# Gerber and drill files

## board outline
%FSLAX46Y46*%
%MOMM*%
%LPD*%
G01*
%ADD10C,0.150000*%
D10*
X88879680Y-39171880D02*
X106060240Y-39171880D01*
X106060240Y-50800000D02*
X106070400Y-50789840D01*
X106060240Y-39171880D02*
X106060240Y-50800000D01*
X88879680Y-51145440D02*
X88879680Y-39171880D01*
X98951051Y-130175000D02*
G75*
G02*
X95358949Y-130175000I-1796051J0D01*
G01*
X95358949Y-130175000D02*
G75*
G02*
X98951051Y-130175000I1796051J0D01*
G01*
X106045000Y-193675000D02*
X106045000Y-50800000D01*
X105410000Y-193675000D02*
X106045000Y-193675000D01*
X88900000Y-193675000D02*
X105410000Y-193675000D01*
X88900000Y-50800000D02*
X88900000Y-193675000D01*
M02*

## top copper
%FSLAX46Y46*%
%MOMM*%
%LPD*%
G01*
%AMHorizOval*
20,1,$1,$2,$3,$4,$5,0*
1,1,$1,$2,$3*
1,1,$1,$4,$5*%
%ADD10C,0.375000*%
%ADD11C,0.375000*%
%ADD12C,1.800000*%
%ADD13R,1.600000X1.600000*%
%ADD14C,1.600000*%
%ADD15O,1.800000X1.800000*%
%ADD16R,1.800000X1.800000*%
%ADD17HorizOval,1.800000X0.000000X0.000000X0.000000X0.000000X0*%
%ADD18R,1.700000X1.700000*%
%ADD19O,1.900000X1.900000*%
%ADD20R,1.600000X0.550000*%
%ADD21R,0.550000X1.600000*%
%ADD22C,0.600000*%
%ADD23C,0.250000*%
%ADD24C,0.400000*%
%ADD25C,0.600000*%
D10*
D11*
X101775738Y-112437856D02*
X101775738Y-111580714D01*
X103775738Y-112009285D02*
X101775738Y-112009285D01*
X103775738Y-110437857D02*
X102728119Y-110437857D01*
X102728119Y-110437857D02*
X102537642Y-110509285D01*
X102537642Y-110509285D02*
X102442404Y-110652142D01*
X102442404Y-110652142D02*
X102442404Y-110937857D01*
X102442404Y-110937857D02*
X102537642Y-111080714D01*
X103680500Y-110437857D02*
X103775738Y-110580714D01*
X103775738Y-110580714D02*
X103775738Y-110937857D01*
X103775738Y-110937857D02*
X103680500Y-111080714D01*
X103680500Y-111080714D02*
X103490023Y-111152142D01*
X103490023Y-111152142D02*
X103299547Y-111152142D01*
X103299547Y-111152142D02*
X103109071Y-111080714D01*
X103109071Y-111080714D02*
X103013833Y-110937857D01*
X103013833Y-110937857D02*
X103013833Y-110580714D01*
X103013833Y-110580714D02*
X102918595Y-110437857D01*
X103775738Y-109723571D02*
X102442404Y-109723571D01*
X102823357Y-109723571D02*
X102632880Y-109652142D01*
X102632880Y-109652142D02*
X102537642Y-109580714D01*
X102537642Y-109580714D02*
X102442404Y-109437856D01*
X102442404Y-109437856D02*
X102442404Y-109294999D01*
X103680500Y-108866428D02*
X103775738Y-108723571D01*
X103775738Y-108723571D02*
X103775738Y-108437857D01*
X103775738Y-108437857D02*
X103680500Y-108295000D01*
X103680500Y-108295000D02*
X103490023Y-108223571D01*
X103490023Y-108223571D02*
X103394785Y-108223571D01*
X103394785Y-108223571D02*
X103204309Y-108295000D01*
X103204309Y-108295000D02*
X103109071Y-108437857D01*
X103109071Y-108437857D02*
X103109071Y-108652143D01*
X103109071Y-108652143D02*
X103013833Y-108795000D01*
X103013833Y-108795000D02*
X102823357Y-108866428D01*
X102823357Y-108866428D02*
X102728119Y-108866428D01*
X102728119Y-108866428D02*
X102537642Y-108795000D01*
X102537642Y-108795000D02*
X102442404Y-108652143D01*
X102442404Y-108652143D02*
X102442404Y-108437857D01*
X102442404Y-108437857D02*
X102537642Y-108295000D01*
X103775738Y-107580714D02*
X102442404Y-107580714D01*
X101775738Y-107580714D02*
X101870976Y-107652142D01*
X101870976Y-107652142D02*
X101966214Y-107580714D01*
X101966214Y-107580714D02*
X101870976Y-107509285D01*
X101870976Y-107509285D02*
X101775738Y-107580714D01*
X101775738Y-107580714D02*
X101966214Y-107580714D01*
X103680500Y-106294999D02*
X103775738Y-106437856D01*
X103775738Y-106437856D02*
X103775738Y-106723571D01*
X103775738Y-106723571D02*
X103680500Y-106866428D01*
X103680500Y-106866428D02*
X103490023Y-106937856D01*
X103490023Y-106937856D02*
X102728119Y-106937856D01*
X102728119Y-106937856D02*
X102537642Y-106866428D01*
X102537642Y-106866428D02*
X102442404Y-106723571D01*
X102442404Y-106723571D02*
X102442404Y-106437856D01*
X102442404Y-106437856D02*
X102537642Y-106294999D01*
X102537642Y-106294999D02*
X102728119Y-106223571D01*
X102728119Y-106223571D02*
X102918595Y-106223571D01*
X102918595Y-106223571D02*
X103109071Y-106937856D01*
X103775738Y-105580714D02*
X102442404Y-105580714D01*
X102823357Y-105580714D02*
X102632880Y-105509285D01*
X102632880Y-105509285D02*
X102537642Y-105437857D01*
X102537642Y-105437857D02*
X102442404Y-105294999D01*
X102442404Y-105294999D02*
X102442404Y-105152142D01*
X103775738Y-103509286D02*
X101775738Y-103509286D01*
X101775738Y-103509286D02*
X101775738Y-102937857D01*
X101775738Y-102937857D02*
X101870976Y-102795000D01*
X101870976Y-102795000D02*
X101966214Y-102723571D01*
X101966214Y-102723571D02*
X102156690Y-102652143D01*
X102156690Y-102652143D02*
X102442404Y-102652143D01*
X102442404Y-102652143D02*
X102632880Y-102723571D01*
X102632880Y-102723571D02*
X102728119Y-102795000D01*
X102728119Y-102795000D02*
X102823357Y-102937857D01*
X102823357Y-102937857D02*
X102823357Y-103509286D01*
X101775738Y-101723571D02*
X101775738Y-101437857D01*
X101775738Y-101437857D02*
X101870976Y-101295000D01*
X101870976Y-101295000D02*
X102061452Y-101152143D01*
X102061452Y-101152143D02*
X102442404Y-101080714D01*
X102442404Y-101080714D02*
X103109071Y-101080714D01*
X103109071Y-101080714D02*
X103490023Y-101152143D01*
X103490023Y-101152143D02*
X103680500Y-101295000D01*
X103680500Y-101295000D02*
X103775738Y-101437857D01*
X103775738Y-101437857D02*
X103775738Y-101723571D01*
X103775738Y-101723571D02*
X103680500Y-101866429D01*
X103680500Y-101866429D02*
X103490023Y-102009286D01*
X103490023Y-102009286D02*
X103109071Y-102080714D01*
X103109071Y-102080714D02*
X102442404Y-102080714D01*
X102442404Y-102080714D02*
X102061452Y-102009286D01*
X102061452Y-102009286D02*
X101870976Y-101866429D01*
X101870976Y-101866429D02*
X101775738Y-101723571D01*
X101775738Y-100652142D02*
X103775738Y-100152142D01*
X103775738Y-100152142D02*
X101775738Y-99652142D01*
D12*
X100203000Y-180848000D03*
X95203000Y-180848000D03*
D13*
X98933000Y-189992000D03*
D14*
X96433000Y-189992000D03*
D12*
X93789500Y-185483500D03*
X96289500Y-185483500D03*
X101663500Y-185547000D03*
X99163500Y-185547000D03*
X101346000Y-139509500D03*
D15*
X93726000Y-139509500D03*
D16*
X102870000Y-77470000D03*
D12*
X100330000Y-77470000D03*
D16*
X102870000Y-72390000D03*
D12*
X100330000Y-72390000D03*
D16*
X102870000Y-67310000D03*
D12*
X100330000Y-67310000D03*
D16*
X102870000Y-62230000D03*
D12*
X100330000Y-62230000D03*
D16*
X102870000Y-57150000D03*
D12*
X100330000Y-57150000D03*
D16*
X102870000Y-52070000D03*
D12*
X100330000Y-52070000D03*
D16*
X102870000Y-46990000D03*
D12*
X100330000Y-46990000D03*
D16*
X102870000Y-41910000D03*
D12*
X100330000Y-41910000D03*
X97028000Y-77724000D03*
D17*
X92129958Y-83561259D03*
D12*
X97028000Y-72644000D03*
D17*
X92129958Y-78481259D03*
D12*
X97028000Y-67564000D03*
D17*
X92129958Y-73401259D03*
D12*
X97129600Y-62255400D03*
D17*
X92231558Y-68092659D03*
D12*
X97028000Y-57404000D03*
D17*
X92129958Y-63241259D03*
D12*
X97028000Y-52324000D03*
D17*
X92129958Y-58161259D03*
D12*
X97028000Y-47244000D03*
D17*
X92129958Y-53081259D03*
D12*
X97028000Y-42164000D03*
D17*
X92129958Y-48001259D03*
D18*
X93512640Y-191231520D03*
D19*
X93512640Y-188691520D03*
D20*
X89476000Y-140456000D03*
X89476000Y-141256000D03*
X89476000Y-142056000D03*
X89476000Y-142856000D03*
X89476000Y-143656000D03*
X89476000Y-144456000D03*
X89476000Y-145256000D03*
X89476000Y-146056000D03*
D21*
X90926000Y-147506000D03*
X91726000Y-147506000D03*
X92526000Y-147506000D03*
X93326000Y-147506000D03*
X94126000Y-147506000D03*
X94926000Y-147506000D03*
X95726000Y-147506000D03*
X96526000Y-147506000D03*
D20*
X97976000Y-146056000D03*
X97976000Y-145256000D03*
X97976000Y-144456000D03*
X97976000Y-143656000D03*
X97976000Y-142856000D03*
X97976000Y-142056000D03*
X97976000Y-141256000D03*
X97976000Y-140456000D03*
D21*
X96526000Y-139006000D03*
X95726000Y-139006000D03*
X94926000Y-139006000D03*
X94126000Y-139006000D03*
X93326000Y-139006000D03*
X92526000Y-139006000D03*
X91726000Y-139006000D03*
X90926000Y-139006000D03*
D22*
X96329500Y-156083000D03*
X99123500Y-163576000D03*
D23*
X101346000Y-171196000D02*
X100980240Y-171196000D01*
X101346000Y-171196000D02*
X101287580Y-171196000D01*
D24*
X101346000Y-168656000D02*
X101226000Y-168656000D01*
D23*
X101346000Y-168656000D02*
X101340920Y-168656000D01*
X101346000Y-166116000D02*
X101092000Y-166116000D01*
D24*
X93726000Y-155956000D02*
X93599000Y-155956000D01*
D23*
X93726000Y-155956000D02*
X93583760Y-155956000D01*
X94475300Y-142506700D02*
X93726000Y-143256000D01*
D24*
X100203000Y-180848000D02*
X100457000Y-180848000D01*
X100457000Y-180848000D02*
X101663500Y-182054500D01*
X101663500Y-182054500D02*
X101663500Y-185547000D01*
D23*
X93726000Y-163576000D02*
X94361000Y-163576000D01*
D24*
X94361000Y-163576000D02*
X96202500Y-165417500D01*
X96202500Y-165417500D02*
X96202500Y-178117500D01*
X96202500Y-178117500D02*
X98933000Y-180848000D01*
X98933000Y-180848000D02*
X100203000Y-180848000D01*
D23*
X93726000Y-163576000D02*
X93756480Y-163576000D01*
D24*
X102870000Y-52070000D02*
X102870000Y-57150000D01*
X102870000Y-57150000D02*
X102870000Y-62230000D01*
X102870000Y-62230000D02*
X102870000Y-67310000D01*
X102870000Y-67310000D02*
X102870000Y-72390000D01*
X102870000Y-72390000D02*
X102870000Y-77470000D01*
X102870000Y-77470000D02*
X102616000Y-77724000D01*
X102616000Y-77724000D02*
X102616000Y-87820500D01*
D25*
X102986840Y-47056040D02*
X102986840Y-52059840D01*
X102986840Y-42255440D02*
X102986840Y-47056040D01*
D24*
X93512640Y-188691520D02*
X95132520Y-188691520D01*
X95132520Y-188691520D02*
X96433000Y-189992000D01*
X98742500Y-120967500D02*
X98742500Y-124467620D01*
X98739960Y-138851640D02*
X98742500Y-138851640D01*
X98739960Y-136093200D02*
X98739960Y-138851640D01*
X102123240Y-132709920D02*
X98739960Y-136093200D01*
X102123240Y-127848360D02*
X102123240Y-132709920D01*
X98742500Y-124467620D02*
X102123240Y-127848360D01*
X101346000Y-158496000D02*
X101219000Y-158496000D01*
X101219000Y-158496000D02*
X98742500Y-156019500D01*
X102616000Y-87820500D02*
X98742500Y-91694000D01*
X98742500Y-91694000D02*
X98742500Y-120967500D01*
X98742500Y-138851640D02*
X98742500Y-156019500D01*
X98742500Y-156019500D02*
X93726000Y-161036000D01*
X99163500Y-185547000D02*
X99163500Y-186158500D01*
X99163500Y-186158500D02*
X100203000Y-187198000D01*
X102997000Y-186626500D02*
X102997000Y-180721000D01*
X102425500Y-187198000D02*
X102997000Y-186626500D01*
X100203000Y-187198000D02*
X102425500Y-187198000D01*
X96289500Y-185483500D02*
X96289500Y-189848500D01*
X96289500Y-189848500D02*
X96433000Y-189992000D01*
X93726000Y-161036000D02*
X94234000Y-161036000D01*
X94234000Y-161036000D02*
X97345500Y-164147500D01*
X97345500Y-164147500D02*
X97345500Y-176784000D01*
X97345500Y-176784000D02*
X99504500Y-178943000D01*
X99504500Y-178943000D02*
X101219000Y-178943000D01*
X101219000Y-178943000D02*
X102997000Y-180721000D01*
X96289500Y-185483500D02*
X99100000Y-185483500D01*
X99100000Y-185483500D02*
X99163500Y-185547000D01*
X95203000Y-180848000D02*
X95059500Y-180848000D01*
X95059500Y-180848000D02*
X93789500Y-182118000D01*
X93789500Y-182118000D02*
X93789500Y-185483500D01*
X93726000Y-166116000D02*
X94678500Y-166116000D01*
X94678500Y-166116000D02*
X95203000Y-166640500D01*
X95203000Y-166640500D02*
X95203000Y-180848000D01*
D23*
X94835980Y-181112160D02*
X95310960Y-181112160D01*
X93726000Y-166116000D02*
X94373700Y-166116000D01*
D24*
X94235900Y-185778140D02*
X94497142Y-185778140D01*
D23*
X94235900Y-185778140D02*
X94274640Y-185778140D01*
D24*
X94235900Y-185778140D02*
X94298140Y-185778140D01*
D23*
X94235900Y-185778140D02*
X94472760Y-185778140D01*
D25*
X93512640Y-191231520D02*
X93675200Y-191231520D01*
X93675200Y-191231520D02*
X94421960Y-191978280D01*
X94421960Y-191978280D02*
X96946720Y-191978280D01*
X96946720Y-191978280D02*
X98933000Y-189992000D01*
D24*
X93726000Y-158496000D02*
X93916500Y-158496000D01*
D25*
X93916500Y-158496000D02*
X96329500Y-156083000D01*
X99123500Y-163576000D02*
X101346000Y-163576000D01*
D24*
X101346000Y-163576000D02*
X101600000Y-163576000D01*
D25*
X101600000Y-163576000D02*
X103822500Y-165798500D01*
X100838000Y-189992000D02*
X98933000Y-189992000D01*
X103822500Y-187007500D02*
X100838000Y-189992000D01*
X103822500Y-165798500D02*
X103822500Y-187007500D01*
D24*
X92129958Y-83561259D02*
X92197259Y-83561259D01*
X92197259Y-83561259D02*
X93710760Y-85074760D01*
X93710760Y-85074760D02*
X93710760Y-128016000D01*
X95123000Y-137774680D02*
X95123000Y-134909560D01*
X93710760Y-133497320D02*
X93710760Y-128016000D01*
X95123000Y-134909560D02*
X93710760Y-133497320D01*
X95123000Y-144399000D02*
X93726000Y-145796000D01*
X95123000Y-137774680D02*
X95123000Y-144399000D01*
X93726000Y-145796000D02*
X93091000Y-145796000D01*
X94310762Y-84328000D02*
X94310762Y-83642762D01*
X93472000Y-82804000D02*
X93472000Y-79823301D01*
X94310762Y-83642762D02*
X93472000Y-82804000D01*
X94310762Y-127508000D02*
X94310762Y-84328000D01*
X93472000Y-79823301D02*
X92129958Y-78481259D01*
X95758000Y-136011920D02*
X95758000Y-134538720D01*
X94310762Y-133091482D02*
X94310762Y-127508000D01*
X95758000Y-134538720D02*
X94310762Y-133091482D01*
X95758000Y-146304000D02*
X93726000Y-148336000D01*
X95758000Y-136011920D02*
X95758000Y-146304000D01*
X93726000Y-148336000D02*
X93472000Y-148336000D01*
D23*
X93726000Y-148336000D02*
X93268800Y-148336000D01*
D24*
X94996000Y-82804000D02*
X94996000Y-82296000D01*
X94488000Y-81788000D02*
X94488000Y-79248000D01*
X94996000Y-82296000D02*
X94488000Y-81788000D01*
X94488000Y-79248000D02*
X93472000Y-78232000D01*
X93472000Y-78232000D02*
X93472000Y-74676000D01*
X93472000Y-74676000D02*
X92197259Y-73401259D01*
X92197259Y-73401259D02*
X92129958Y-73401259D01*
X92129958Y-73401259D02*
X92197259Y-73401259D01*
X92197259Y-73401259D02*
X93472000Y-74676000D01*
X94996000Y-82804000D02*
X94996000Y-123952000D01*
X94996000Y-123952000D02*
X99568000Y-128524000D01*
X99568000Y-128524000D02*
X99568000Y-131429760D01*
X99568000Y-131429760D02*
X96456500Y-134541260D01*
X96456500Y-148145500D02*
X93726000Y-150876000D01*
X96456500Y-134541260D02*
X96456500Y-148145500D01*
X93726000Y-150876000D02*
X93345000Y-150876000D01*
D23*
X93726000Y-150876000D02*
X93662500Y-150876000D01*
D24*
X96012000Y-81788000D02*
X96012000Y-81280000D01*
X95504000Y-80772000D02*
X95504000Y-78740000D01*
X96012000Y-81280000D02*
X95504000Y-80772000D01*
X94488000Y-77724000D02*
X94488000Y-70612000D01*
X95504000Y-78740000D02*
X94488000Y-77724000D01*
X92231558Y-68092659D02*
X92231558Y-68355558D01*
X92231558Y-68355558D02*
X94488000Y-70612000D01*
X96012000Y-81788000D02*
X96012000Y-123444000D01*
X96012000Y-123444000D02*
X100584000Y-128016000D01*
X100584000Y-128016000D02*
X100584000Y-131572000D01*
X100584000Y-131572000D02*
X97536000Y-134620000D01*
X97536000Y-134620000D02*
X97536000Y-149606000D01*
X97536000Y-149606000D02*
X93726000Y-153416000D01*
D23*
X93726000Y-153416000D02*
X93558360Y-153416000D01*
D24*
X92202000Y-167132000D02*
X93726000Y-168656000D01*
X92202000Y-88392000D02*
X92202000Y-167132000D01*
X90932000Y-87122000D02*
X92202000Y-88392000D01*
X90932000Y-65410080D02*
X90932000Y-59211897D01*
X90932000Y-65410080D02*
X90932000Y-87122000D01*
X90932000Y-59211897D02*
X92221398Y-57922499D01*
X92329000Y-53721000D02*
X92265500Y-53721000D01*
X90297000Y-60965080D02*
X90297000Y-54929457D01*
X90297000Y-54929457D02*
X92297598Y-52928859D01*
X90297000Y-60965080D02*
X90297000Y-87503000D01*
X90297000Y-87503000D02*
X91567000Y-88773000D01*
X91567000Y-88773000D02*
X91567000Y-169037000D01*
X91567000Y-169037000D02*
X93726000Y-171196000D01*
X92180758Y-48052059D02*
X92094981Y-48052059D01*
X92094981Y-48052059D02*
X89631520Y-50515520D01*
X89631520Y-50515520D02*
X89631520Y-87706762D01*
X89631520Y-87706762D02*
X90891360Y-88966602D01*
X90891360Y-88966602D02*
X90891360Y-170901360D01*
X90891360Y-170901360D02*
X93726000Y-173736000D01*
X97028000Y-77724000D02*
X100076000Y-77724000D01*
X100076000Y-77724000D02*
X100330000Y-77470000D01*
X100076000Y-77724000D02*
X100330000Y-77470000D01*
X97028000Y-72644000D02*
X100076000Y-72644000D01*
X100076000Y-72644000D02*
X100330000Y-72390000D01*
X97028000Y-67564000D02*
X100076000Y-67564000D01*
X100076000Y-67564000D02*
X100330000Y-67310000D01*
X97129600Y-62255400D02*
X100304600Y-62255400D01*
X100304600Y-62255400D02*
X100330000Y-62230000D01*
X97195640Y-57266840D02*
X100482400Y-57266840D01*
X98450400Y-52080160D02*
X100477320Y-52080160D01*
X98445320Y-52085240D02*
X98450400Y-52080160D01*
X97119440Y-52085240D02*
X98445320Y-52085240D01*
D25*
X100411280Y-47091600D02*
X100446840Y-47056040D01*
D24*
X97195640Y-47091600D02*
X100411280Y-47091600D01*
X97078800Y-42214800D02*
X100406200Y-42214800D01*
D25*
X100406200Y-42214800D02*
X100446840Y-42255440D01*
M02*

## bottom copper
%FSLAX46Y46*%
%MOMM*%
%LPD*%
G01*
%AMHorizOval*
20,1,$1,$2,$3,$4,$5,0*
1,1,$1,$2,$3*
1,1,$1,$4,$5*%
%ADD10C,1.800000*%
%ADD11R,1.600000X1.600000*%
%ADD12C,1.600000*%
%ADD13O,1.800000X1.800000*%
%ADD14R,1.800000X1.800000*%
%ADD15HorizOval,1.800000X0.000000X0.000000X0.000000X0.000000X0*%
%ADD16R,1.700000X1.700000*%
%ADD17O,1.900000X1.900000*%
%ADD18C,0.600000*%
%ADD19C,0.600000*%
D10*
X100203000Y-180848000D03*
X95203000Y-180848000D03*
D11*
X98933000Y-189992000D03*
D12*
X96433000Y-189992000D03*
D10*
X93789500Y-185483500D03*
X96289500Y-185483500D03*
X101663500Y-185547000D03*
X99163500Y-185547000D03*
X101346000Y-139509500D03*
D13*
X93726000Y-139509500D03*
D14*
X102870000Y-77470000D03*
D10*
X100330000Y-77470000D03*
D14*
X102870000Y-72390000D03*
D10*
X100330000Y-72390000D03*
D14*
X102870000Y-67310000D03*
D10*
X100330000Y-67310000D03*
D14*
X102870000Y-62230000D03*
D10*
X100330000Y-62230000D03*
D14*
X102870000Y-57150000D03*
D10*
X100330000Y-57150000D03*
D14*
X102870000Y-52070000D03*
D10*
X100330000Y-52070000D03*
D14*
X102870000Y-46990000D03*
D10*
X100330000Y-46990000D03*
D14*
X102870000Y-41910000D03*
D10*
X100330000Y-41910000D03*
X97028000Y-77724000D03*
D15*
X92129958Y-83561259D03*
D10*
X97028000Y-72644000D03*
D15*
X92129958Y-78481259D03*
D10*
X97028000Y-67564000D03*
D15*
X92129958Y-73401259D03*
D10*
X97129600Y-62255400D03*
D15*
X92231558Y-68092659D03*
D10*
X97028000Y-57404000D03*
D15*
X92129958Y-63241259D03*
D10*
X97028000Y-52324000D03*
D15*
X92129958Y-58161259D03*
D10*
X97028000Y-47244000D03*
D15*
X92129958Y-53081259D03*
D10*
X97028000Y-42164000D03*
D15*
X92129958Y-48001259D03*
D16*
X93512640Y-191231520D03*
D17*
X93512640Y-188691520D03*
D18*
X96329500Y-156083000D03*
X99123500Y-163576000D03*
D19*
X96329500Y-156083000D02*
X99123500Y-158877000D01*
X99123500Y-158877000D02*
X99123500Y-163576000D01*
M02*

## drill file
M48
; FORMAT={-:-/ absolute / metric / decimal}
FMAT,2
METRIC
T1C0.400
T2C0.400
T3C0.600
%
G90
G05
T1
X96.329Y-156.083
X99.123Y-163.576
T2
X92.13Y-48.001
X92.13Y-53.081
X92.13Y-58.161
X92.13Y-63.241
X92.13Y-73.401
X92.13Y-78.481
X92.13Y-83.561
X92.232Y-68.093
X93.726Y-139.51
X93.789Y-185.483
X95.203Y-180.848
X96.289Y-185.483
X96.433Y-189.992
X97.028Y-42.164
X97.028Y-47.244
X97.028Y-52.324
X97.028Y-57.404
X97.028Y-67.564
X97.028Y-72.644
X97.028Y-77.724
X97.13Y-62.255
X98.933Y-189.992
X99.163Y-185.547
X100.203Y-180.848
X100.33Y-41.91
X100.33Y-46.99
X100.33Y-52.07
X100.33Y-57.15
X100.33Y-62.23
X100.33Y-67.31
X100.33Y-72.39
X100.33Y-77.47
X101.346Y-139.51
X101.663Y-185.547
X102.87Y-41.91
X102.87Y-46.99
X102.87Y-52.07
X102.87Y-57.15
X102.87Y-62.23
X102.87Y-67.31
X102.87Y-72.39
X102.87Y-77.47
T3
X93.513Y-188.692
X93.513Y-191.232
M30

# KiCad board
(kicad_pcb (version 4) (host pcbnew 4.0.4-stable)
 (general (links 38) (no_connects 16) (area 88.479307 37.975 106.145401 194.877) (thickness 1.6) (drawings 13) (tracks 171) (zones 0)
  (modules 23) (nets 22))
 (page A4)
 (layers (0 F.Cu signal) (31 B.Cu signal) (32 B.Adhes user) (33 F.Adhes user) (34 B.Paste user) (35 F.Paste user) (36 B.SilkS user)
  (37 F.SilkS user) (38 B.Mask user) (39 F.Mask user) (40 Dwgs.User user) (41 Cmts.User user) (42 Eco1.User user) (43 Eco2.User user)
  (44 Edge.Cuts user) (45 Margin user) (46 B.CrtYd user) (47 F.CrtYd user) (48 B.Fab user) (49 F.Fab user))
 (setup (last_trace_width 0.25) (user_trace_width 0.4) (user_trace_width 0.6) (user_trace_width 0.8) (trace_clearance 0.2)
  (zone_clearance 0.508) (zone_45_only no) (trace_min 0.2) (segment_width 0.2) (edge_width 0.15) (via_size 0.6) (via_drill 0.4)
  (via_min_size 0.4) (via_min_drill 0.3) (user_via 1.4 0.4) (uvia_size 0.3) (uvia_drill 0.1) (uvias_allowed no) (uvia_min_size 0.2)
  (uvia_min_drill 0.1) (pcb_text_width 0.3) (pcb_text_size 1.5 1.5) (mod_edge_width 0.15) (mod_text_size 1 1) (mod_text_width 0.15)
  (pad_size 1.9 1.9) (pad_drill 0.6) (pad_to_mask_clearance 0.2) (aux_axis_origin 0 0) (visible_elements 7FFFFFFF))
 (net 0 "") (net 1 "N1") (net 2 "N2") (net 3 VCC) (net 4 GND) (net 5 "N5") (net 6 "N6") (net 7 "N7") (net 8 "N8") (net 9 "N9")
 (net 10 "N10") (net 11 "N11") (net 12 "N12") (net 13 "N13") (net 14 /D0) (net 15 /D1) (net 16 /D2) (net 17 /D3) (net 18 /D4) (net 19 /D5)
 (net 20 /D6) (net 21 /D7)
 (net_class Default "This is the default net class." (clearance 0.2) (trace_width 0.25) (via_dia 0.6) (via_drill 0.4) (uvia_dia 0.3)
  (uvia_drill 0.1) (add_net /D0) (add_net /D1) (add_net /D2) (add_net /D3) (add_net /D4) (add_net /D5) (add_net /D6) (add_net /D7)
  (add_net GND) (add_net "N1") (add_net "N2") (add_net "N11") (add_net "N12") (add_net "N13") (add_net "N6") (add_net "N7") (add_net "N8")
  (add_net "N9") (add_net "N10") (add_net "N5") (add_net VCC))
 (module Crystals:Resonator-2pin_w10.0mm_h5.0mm (layer F.Cu) (at 100.203 180.848 180)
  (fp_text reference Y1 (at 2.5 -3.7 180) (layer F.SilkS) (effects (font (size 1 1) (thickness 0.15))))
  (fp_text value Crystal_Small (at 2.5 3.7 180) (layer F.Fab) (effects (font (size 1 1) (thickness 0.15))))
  (pad 1 thru_hole circle (at 0 0 180) (size 1.8 1.8) (drill 0.4) (layers *.Cu *.Mask) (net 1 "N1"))
  (pad 2 thru_hole circle (at 5 0 180) (size 1.8 1.8) (drill 0.4) (layers *.Cu *.Mask) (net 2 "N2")))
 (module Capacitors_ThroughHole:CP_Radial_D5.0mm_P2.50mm (layer F.Cu) (at 98.933 189.992 180)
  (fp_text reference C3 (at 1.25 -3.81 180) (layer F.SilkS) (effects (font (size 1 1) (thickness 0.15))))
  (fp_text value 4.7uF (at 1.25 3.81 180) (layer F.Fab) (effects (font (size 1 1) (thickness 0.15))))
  (pad 1 thru_hole rect (at 0 0 180) (size 1.6 1.6) (drill 0.4) (layers *.Cu *.Mask) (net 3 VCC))
  (pad 2 thru_hole circle (at 2.5 0 180) (size 1.6 1.6) (drill 0.4) (layers *.Cu *.Mask) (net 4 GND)))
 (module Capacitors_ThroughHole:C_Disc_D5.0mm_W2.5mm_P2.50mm (layer F.Cu) (at 93.7895 185.4835)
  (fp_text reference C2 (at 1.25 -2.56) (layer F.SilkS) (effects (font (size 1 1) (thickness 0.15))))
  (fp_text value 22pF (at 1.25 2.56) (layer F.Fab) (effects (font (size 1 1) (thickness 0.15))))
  (pad 1 thru_hole circle (at 0 0) (size 1.8 1.8) (drill 0.4) (layers *.Cu *.Mask) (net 2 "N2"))
  (pad 2 thru_hole circle (at 2.5 0) (size 1.8 1.8) (drill 0.4) (layers *.Cu *.Mask) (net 4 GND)))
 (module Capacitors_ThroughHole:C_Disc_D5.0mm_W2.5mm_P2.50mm (layer F.Cu) (at 101.6635 185.547 180)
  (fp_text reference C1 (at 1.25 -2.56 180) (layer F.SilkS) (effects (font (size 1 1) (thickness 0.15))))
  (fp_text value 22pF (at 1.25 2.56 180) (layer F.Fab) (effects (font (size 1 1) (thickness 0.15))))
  (pad 1 thru_hole circle (at 0 0 180) (size 1.8 1.8) (drill 0.4) (layers *.Cu *.Mask) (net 1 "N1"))
  (pad 2 thru_hole circle (at 2.5 0 180) (size 1.8 1.8) (drill 0.4) (layers *.Cu *.Mask) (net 4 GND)))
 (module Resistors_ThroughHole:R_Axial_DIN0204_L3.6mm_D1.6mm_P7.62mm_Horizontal (layer F.Cu) (at 101.346 139.5095 180)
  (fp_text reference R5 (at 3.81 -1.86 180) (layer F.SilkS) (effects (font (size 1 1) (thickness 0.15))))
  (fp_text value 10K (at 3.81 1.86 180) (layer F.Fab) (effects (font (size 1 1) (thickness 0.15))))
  (pad 1 thru_hole circle (at 0 0 180) (size 1.8 1.8) (drill 0.4) (layers *.Cu *.Mask) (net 3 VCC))
  (pad 2 thru_hole oval (at 7.62 0 180) (size 1.8 1.8) (drill 0.4) (layers *.Cu *.Mask) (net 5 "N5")))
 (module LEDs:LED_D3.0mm (layer F.Cu) (at 102.87 77.47 180)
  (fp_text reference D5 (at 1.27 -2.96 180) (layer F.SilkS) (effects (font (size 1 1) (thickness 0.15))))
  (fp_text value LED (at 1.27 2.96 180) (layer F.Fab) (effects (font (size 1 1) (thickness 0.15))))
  (pad 1 thru_hole rect (at 0 0 180) (size 1.8 1.8) (drill 0.4) (layers *.Cu *.Mask) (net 4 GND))
  (pad 2 thru_hole circle (at 2.54 0 180) (size 1.8 1.8) (drill 0.4) (layers *.Cu *.Mask) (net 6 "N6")))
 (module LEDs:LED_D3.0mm (layer F.Cu) (at 102.87 72.39 180)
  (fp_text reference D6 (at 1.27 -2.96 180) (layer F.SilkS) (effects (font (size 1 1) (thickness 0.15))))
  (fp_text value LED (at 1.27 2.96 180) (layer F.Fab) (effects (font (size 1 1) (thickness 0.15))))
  (pad 1 thru_hole rect (at 0 0 180) (size 1.8 1.8) (drill 0.4) (layers *.Cu *.Mask) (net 4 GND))
  (pad 2 thru_hole circle (at 2.54 0 180) (size 1.8 1.8) (drill 0.4) (layers *.Cu *.Mask) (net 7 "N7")))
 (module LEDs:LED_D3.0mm (layer F.Cu) (at 102.87 67.31 180)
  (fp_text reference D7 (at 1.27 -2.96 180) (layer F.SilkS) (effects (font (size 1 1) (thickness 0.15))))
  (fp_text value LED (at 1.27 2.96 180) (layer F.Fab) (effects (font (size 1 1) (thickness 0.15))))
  (pad 1 thru_hole rect (at 0 0 180) (size 1.8 1.8) (drill 0.4) (layers *.Cu *.Mask) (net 4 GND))
  (pad 2 thru_hole circle (at 2.54 0 180) (size 1.8 1.8) (drill 0.4) (layers *.Cu *.Mask) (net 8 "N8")))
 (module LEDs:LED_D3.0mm (layer F.Cu) (at 102.87 62.23 180)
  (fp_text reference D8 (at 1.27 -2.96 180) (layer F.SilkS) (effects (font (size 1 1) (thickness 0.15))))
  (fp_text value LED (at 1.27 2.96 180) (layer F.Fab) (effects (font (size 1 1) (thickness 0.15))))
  (pad 1 thru_hole rect (at 0 0 180) (size 1.8 1.8) (drill 0.4) (layers *.Cu *.Mask) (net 4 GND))
  (pad 2 thru_hole circle (at 2.54 0 180) (size 1.8 1.8) (drill 0.4) (layers *.Cu *.Mask) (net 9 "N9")))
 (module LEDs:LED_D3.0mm (layer F.Cu) (at 102.87 57.15 180)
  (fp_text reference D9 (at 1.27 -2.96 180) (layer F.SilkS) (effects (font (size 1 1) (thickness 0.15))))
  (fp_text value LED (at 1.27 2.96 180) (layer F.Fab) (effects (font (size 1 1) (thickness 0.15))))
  (pad 1 thru_hole rect (at 0 0 180) (size 1.8 1.8) (drill 0.4) (layers *.Cu *.Mask) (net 4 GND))
  (pad 2 thru_hole circle (at 2.54 0 180) (size 1.8 1.8) (drill 0.4) (layers *.Cu *.Mask) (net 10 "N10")))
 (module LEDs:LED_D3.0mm (layer F.Cu) (at 102.87 52.07 180)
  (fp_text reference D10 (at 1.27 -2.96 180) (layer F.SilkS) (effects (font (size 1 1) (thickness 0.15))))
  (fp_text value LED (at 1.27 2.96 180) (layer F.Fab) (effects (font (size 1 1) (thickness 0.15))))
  (pad 1 thru_hole rect (at 0 0 180) (size 1.8 1.8) (drill 0.4) (layers *.Cu *.Mask) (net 4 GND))
  (pad 2 thru_hole circle (at 2.54 0 180) (size 1.8 1.8) (drill 0.4) (layers *.Cu *.Mask) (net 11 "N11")))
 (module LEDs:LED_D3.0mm (layer F.Cu) (at 102.87 46.99 180)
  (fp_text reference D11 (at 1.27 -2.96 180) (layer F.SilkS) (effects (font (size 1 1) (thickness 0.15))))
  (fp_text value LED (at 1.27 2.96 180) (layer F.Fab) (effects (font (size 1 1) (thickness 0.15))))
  (pad 1 thru_hole rect (at 0 0 180) (size 1.8 1.8) (drill 0.4) (layers *.Cu *.Mask) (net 4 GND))
  (pad 2 thru_hole circle (at 2.54 0 180) (size 1.8 1.8) (drill 0.4) (layers *.Cu *.Mask) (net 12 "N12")))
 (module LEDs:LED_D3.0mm (layer F.Cu) (at 102.87 41.91 180)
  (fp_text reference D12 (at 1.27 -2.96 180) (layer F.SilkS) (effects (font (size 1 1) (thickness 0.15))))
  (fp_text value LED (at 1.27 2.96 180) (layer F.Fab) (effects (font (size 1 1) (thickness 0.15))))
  (pad 1 thru_hole rect (at 0 0 180) (size 1.8 1.8) (drill 0.4) (layers *.Cu *.Mask) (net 4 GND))
  (pad 2 thru_hole circle (at 2.54 0 180) (size 1.8 1.8) (drill 0.4) (layers *.Cu *.Mask) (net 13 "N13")))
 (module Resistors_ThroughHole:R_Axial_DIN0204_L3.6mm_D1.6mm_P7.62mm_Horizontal (layer F.Cu) (at 97.028 77.724 230)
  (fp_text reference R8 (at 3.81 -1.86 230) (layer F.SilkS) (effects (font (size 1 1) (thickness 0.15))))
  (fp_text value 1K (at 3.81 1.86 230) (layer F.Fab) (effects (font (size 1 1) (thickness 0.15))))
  (pad 1 thru_hole circle (at 0 0 230) (size 1.8 1.8) (drill 0.4) (layers *.Cu *.Mask) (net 6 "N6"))
  (pad 2 thru_hole oval (at 7.62 0 230) (size 1.8 1.8) (drill 0.4) (layers *.Cu *.Mask) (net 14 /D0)))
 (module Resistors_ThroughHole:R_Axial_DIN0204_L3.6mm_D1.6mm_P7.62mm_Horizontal (layer F.Cu) (at 97.028 72.644 230)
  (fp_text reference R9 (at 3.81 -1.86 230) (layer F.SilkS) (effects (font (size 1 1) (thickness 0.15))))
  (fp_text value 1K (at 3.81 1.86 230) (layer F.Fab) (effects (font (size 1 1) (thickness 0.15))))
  (pad 1 thru_hole circle (at 0 0 230) (size 1.8 1.8) (drill 0.4) (layers *.Cu *.Mask) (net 7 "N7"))
  (pad 2 thru_hole oval (at 7.62 0 230) (size 1.8 1.8) (drill 0.4) (layers *.Cu *.Mask) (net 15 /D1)))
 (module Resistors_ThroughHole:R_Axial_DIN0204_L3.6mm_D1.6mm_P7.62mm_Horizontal (layer F.Cu) (at 97.028 67.564 230)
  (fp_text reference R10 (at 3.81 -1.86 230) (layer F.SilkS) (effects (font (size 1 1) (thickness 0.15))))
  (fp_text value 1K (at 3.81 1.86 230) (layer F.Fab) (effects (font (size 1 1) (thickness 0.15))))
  (pad 1 thru_hole circle (at 0 0 230) (size 1.8 1.8) (drill 0.4) (layers *.Cu *.Mask) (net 8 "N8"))
  (pad 2 thru_hole oval (at 7.62 0 230) (size 1.8 1.8) (drill 0.4) (layers *.Cu *.Mask) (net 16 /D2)))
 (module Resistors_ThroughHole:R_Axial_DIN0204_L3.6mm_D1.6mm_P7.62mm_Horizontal (layer F.Cu) (at 97.1296 62.2554 230)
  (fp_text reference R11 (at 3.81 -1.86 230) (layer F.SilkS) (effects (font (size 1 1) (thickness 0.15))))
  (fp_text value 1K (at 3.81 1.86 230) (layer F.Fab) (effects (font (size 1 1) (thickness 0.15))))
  (pad 1 thru_hole circle (at 0 0 230) (size 1.8 1.8) (drill 0.4) (layers *.Cu *.Mask) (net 9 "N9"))
  (pad 2 thru_hole oval (at 7.62 0 230) (size 1.8 1.8) (drill 0.4) (layers *.Cu *.Mask) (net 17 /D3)))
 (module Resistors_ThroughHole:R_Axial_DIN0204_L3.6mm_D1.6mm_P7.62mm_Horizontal (layer F.Cu) (at 97.028 57.404 230)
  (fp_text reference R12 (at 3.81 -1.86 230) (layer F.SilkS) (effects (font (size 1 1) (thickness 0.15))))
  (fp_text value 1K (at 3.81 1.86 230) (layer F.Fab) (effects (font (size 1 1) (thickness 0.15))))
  (pad 1 thru_hole circle (at 0 0 230) (size 1.8 1.8) (drill 0.4) (layers *.Cu *.Mask) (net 10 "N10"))
  (pad 2 thru_hole oval (at 7.62 0 230) (size 1.8 1.8) (drill 0.4) (layers *.Cu *.Mask) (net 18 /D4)))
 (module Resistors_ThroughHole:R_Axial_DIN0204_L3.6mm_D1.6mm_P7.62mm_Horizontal (layer F.Cu) (at 97.028 52.324 230)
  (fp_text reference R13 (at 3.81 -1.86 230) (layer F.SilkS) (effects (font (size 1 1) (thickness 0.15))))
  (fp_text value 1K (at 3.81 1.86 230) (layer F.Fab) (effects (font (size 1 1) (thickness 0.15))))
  (pad 1 thru_hole circle (at 0 0 230) (size 1.8 1.8) (drill 0.4) (layers *.Cu *.Mask) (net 11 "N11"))
  (pad 2 thru_hole oval (at 7.62 0 230) (size 1.8 1.8) (drill 0.4) (layers *.Cu *.Mask) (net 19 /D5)))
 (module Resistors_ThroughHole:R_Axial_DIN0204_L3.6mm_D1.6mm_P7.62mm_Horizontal (layer F.Cu) (at 97.028 47.244 230)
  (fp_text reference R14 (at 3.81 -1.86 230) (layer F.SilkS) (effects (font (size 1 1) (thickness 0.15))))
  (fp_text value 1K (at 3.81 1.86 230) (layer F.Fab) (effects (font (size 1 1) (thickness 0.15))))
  (pad 1 thru_hole circle (at 0 0 230) (size 1.8 1.8) (drill 0.4) (layers *.Cu *.Mask) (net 12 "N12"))
  (pad 2 thru_hole oval (at 7.62 0 230) (size 1.8 1.8) (drill 0.4) (layers *.Cu *.Mask) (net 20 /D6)))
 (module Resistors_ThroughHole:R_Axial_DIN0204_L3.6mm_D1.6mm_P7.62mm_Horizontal (layer F.Cu) (at 97.028 42.164 230)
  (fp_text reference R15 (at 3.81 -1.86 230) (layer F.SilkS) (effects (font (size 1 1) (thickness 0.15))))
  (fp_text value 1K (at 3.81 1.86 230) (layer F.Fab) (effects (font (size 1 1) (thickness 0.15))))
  (pad 1 thru_hole circle (at 0 0 230) (size 1.8 1.8) (drill 0.4) (layers *.Cu *.Mask) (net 13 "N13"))
  (pad 2 thru_hole oval (at 7.62 0 230) (size 1.8 1.8) (drill 0.4) (layers *.Cu *.Mask) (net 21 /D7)))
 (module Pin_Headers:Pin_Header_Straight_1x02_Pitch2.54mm (layer F.Cu) (at 93.51264 191.23152 180)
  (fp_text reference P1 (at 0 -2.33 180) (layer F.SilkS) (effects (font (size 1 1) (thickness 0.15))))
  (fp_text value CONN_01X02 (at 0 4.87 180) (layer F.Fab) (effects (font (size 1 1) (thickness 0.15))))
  (pad 1 thru_hole rect (at 0 0 180) (size 1.7 1.7) (drill 0.6) (layers *.Cu *.Mask) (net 3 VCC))
  (pad 2 thru_hole oval (at 0 2.54 180) (size 1.9 1.9) (drill 0.6) (layers *.Cu *.Mask) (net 4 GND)))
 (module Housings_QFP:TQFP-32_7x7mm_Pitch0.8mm (layer F.Cu) (at 93.726 143.256)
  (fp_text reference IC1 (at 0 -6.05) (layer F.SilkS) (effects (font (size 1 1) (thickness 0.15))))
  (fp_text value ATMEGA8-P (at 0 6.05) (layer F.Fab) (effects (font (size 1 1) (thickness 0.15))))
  (pad 1 smd rect (at -4.25 -2.8) (size 1.6 0.55) (layers F.Cu F.Paste F.Mask) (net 5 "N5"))
  (pad 2 smd rect (at -4.25 -2) (size 1.6 0.55) (layers F.Cu F.Paste F.Mask) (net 14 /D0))
  (pad 3 smd rect (at -4.25 -1.2) (size 1.6 0.55) (layers F.Cu F.Paste F.Mask) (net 15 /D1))
  (pad 4 smd rect (at -4.25 -0.4) (size 1.6 0.55) (layers F.Cu F.Paste F.Mask) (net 16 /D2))
  (pad 5 smd rect (at -4.25 0.4) (size 1.6 0.55) (layers F.Cu F.Paste F.Mask) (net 17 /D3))
  (pad 6 smd rect (at -4.25 1.2) (size 1.6 0.55) (layers F.Cu F.Paste F.Mask) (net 18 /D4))
  (pad 7 smd rect (at -4.25 2) (size 1.6 0.55) (layers F.Cu F.Paste F.Mask) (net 3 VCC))
  (pad 8 smd rect (at -4.25 2.8) (size 1.6 0.55) (layers F.Cu F.Paste F.Mask) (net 4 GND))
  (pad 9 smd rect (at -2.8 4.25 90) (size 1.6 0.55) (layers F.Cu F.Paste F.Mask) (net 1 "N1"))
  (pad 10 smd rect (at -2 4.25 90) (size 1.6 0.55) (layers F.Cu F.Paste F.Mask) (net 2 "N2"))
  (pad 11 smd rect (at -1.2 4.25 90) (size 1.6 0.55) (layers F.Cu F.Paste F.Mask) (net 19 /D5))
  (pad 12 smd rect (at -0.4 4.25 90) (size 1.6 0.55) (layers F.Cu F.Paste F.Mask) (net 20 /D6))
  (pad 13 smd rect (at 0.4 4.25 90) (size 1.6 0.55) (layers F.Cu F.Paste F.Mask) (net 21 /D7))
  (pad 14 smd rect (at 1.2 4.25 90) (size 1.6 0.55) (layers F.Cu F.Paste F.Mask))
  (pad 15 smd rect (at 2 4.25 90) (size 1.6 0.55) (layers F.Cu F.Paste F.Mask))
  (pad 16 smd rect (at 2.8 4.25 90) (size 1.6 0.55) (layers F.Cu F.Paste F.Mask))
  (pad 17 smd rect (at 4.25 2.8) (size 1.6 0.55) (layers F.Cu F.Paste F.Mask))
  (pad 18 smd rect (at 4.25 2) (size 1.6 0.55) (layers F.Cu F.Paste F.Mask))
  (pad 19 smd rect (at 4.25 1.2) (size 1.6 0.55) (layers F.Cu F.Paste F.Mask))
  (pad 20 smd rect (at 4.25 0.4) (size 1.6 0.55) (layers F.Cu F.Paste F.Mask) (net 3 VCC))
  (pad 21 smd rect (at 4.25 -0.4) (size 1.6 0.55) (layers F.Cu F.Paste F.Mask))
  (pad 22 smd rect (at 4.25 -1.2) (size 1.6 0.55) (layers F.Cu F.Paste F.Mask) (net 4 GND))
  (pad 23 smd rect (at 4.25 -2) (size 1.6 0.55) (layers F.Cu F.Paste F.Mask))
  (pad 24 smd rect (at 4.25 -2.8) (size 1.6 0.55) (layers F.Cu F.Paste F.Mask))
  (pad 25 smd rect (at 2.8 -4.25 90) (size 1.6 0.55) (layers F.Cu F.Paste F.Mask))
  (pad 26 smd rect (at 2 -4.25 90) (size 1.6 0.55) (layers F.Cu F.Paste F.Mask))
  (pad 27 smd rect (at 1.2 -4.25 90) (size 1.6 0.55) (layers F.Cu F.Paste F.Mask))
  (pad 28 smd rect (at 0.4 -4.25 90) (size 1.6 0.55) (layers F.Cu F.Paste F.Mask))
  (pad 29 smd rect (at -0.4 -4.25 90) (size 1.6 0.55) (layers F.Cu F.Paste F.Mask))
  (pad 30 smd rect (at -1.2 -4.25 90) (size 1.6 0.55) (layers F.Cu F.Paste F.Mask))
  (pad 31 smd rect (at -2 -4.25 90) (size 1.6 0.55) (layers F.Cu F.Paste F.Mask))
  (pad 32 smd rect (at -2.8 -4.25 90) (size 1.6 0.55) (layers F.Cu F.Paste F.Mask)))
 (gr_line (start 88.87968 39.17188) (end 106.06024 39.17188) (angle 90) (layer Edge.Cuts) (width 0.15))
 (gr_line (start 106.06024 50.8) (end 106.0704 50.78984) (angle 90) (layer Edge.Cuts) (width 0.15))
 (gr_line (start 106.06024 39.17188) (end 106.06024 50.8) (angle 90) (layer Edge.Cuts) (width 0.15))
 (gr_line (start 88.87968 51.14544) (end 88.87968 39.17188) (angle 90) (layer Edge.Cuts) (width 0.15))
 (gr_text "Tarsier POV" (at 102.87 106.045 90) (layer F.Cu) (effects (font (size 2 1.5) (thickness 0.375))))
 (gr_circle (center 97.155 130.175) (end 98.425 131.445) (layer Edge.Cuts) (width 0.15))
 (gr_line (start 106.045 193.675) (end 106.045 50.8) (angle 90) (layer Edge.Cuts) (width 0.15))
 (gr_line (start 105.41 193.675) (end 106.045 193.675) (angle 90) (layer Edge.Cuts) (width 0.15))
 (gr_line (start 88.9 193.675) (end 105.41 193.675) (angle 90) (layer Edge.Cuts) (width 0.15))
 (gr_line (start 88.9 50.8) (end 88.9 193.675) (angle 90) (layer Edge.Cuts) (width 0.15))
 (segment (start 101.346 171.196) (end 100.98024 171.196) (width 0.25) (layer F.Cu) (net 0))
 (segment (start 101.346 171.196) (end 101.28758 171.196) (width 0.25) (layer F.Cu) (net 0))
 (segment (start 101.346 168.656) (end 101.226 168.656) (width 0.4) (layer F.Cu) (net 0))
 (segment (start 101.346 168.656) (end 101.34092 168.656) (width 0.25) (layer F.Cu) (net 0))
 (segment (start 101.346 166.116) (end 101.092 166.116) (width 0.25) (layer F.Cu) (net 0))
 (segment (start 93.726 155.956) (end 93.599 155.956) (width 0.4) (layer F.Cu) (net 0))
 (segment (start 93.726 155.956) (end 93.58376 155.956) (width 0.25) (layer F.Cu) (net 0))
 (segment (start 94.4753 142.5067) (end 93.726 143.256) (width 0.25) (layer F.Cu) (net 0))
 (segment (start 100.203 180.848) (end 100.457 180.848) (width 0.4) (layer F.Cu) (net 1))
 (segment (start 100.457 180.848) (end 101.6635 182.0545) (width 0.4) (layer F.Cu) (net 1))
 (segment (start 101.6635 182.0545) (end 101.6635 185.547) (width 0.4) (layer F.Cu) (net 1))
 (segment (start 93.726 163.576) (end 94.361 163.576) (width 0.25) (layer F.Cu) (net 1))
 (segment (start 94.361 163.576) (end 96.2025 165.4175) (width 0.4) (layer F.Cu) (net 1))
 (segment (start 96.2025 165.4175) (end 96.2025 178.1175) (width 0.4) (layer F.Cu) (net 1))
 (segment (start 96.2025 178.1175) (end 98.933 180.848) (width 0.4) (layer F.Cu) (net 1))
 (segment (start 98.933 180.848) (end 100.203 180.848) (width 0.4) (layer F.Cu) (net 1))
 (segment (start 93.726 163.576) (end 93.75648 163.576) (width 0.25) (layer F.Cu) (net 1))
 (segment (start 102.87 52.07) (end 102.87 57.15) (width 0.4) (layer F.Cu) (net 4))
 (segment (start 102.87 57.15) (end 102.87 62.23) (width 0.4) (layer F.Cu) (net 4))
 (segment (start 102.87 62.23) (end 102.87 67.31) (width 0.4) (layer F.Cu) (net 4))
 (segment (start 102.87 67.31) (end 102.87 72.39) (width 0.4) (layer F.Cu) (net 4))
 (segment (start 102.87 72.39) (end 102.87 77.47) (width 0.4) (layer F.Cu) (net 4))
 (segment (start 102.87 77.47) (end 102.616 77.724) (width 0.4) (layer F.Cu) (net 4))
 (segment (start 102.616 77.724) (end 102.616 87.8205) (width 0.4) (layer F.Cu) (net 4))
 (segment (start 102.98684 47.05604) (end 102.98684 52.05984) (width 0.6) (layer F.Cu) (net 4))
 (segment (start 102.98684 42.25544) (end 102.98684 47.05604) (width 0.6) (layer F.Cu) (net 4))
 (segment (start 93.51264 188.69152) (end 95.13252 188.69152) (width 0.4) (layer F.Cu) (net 4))
 (segment (start 95.13252 188.69152) (end 96.433 189.992) (width 0.4) (layer F.Cu) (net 4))
 (segment (start 98.7425 120.9675) (end 98.7425 124.46762) (width 0.4) (layer F.Cu) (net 4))
 (segment (start 98.73996 138.85164) (end 98.7425 138.85164) (width 0.4) (layer F.Cu) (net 4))
 (segment (start 98.73996 136.0932) (end 98.73996 138.85164) (width 0.4) (layer F.Cu) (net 4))
 (segment (start 102.12324 132.70992) (end 98.73996 136.0932) (width 0.4) (layer F.Cu) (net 4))
 (segment (start 102.12324 127.84836) (end 102.12324 132.70992) (width 0.4) (layer F.Cu) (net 4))
 (segment (start 98.7425 124.46762) (end 102.12324 127.84836) (width 0.4) (layer F.Cu) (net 4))
 (segment (start 101.346 158.496) (end 101.219 158.496) (width 0.4) (layer F.Cu) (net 4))
 (segment (start 101.219 158.496) (end 98.7425 156.0195) (width 0.4) (layer F.Cu) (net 4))
 (segment (start 102.616 87.8205) (end 98.7425 91.694) (width 0.4) (layer F.Cu) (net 4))
 (segment (start 98.7425 91.694) (end 98.7425 120.9675) (width 0.4) (layer F.Cu) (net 4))
 (segment (start 98.7425 138.85164) (end 98.7425 156.0195) (width 0.4) (layer F.Cu) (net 4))
 (segment (start 98.7425 156.0195) (end 93.726 161.036) (width 0.4) (layer F.Cu) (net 4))
 (segment (start 99.1635 185.547) (end 99.1635 186.1585) (width 0.4) (layer F.Cu) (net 4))
 (segment (start 99.1635 186.1585) (end 100.203 187.198) (width 0.4) (layer F.Cu) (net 4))
 (segment (start 102.997 186.6265) (end 102.997 180.721) (width 0.4) (layer F.Cu) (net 4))
 (segment (start 102.4255 187.198) (end 102.997 186.6265) (width 0.4) (layer F.Cu) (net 4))
 (segment (start 100.203 187.198) (end 102.4255 187.198) (width 0.4) (layer F.Cu) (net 4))
 (segment (start 96.2895 185.4835) (end 96.2895 189.8485) (width 0.4) (layer F.Cu) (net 4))
 (segment (start 96.2895 189.8485) (end 96.433 189.992) (width 0.4) (layer F.Cu) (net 4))
 (segment (start 93.726 161.036) (end 94.234 161.036) (width 0.4) (layer F.Cu) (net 4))
 (segment (start 94.234 161.036) (end 97.3455 164.1475) (width 0.4) (layer F.Cu) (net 4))
 (segment (start 97.3455 164.1475) (end 97.3455 176.784) (width 0.4) (layer F.Cu) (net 4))
 (segment (start 97.3455 176.784) (end 99.5045 178.943) (width 0.4) (layer F.Cu) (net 4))
 (segment (start 99.5045 178.943) (end 101.219 178.943) (width 0.4) (layer F.Cu) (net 4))
 (segment (start 101.219 178.943) (end 102.997 180.721) (width 0.4) (layer F.Cu) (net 4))
 (segment (start 96.2895 185.4835) (end 99.1 185.4835) (width 0.4) (layer F.Cu) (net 4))
 (segment (start 99.1 185.4835) (end 99.1635 185.547) (width 0.4) (layer F.Cu) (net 4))
 (segment (start 95.203 180.848) (end 95.0595 180.848) (width 0.4) (layer F.Cu) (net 2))
 (segment (start 95.0595 180.848) (end 93.7895 182.118) (width 0.4) (layer F.Cu) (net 2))
 (segment (start 93.7895 182.118) (end 93.7895 185.4835) (width 0.4) (layer F.Cu) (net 2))
 (segment (start 93.726 166.116) (end 94.6785 166.116) (width 0.4) (layer F.Cu) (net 2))
 (segment (start 94.6785 166.116) (end 95.203 166.6405) (width 0.4) (layer F.Cu) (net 2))
 (segment (start 95.203 166.6405) (end 95.203 180.848) (width 0.4) (layer F.Cu) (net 2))
 (segment (start 94.83598 181.11216) (end 95.31096 181.11216) (width 0.25) (layer F.Cu) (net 2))
 (segment (start 93.726 166.116) (end 94.3737 166.116) (width 0.25) (layer F.Cu) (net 2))
 (segment (start 94.2359 185.77814) (end 94.497142 185.77814) (width 0.4) (layer F.Cu) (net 2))
 (segment (start 94.2359 185.77814) (end 94.27464 185.77814) (width 0.25) (layer F.Cu) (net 2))
 (segment (start 94.2359 185.77814) (end 94.29814 185.77814) (width 0.4) (layer F.Cu) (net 2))
 (segment (start 94.2359 185.77814) (end 94.47276 185.77814) (width 0.25) (layer F.Cu) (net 2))
 (segment (start 93.51264 191.23152) (end 93.6752 191.23152) (width 0.6) (layer F.Cu) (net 3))
 (segment (start 93.6752 191.23152) (end 94.42196 191.97828) (width 0.6) (layer F.Cu) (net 3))
 (segment (start 94.42196 191.97828) (end 96.94672 191.97828) (width 0.6) (layer F.Cu) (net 3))
 (segment (start 96.94672 191.97828) (end 98.933 189.992) (width 0.6) (layer F.Cu) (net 3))
 (segment (start 93.726 158.496) (end 93.9165 158.496) (width 0.4) (layer F.Cu) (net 3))
 (segment (start 93.9165 158.496) (end 96.3295 156.083) (width 0.6) (layer F.Cu) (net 3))
 (via (at 96.3295 156.083) (size 0.6) (drill 0.4) (layers F.Cu B.Cu) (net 3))
 (segment (start 96.3295 156.083) (end 99.1235 158.877) (width 0.6) (layer B.Cu) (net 3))
 (segment (start 99.1235 158.877) (end 99.1235 163.576) (width 0.6) (layer B.Cu) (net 3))
 (via (at 99.1235 163.576) (size 0.6) (drill 0.4) (layers F.Cu B.Cu) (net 3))
 (segment (start 99.1235 163.576) (end 101.346 163.576) (width 0.6) (layer F.Cu) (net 3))
 (segment (start 101.346 163.576) (end 101.6 163.576) (width 0.4) (layer F.Cu) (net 3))
 (segment (start 101.6 163.576) (end 103.8225 165.7985) (width 0.6) (layer F.Cu) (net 3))
 (segment (start 100.838 189.992) (end 98.933 189.992) (width 0.6) (layer F.Cu) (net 3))
 (segment (start 103.8225 187.0075) (end 100.838 189.992) (width 0.6) (layer F.Cu) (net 3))
 (segment (start 103.8225 165.7985) (end 103.8225 187.0075) (width 0.6) (layer F.Cu) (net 3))
 (segment (start 92.129958 83.561259) (end 92.197259 83.561259) (width 0.4) (layer F.Cu) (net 14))
 (segment (start 92.197259 83.561259) (end 93.71076 85.07476) (width 0.4) (layer F.Cu) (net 14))
 (segment (start 93.71076 85.07476) (end 93.71076 128.016) (width 0.4) (layer F.Cu) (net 14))
 (segment (start 95.123 137.77468) (end 95.123 134.90956) (width 0.4) (layer F.Cu) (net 14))
 (segment (start 93.71076 133.49732) (end 93.71076 128.016) (width 0.4) (layer F.Cu) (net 14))
 (segment (start 95.123 134.90956) (end 93.71076 133.49732) (width 0.4) (layer F.Cu) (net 14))
 (segment (start 95.123 144.399) (end 93.726 145.796) (width 0.4) (layer F.Cu) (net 14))
 (segment (start 95.123 137.77468) (end 95.123 144.399) (width 0.4) (layer F.Cu) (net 14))
 (segment (start 93.726 145.796) (end 93.091 145.796) (width 0.4) (layer F.Cu) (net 14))
 (segment (start 94.310762 84.328) (end 94.310762 83.642762) (width 0.4) (layer F.Cu) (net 15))
 (segment (start 93.472 82.804) (end 93.472 79.823301) (width 0.4) (layer F.Cu) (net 15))
 (segment (start 94.310762 83.642762) (end 93.472 82.804) (width 0.4) (layer F.Cu) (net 15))
 (segment (start 94.310762 127.508) (end 94.310762 84.328) (width 0.4) (layer F.Cu) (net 15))
 (segment (start 93.472 79.823301) (end 92.129958 78.481259) (width 0.4) (layer F.Cu) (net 15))
 (segment (start 95.758 136.01192) (end 95.758 134.53872) (width 0.4) (layer F.Cu) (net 15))
 (segment (start 94.310762 133.091482) (end 94.310762 127.508) (width 0.4) (layer F.Cu) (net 15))
 (segment (start 95.758 134.53872) (end 94.310762 133.091482) (width 0.4) (layer F.Cu) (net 15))
 (segment (start 95.758 146.304) (end 93.726 148.336) (width 0.4) (layer F.Cu) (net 15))
 (segment (start 95.758 136.01192) (end 95.758 146.304) (width 0.4) (layer F.Cu) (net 15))
 (segment (start 93.726 148.336) (end 93.472 148.336) (width 0.4) (layer F.Cu) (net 15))
 (segment (start 93.726 148.336) (end 93.2688 148.336) (width 0.25) (layer F.Cu) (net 15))
 (segment (start 94.996 82.804) (end 94.996 82.296) (width 0.4) (layer F.Cu) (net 16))
 (segment (start 94.488 81.788) (end 94.488 79.248) (width 0.4) (layer F.Cu) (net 16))
 (segment (start 94.996 82.296) (end 94.488 81.788) (width 0.4) (layer F.Cu) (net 16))
 (segment (start 94.488 79.248) (end 93.472 78.232) (width 0.4) (layer F.Cu) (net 16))
 (segment (start 93.472 78.232) (end 93.472 74.676) (width 0.4) (layer F.Cu) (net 16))
 (segment (start 93.472 74.676) (end 92.197259 73.401259) (width 0.4) (layer F.Cu) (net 16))
 (segment (start 92.197259 73.401259) (end 92.129958 73.401259) (width 0.4) (layer F.Cu) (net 16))
 (segment (start 92.129958 73.401259) (end 92.197259 73.401259) (width 0.4) (layer F.Cu) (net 16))
 (segment (start 92.197259 73.401259) (end 93.472 74.676) (width 0.4) (layer F.Cu) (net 16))
 (segment (start 94.996 82.804) (end 94.996 123.952) (width 0.4) (layer F.Cu) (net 16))
 (segment (start 94.996 123.952) (end 99.568 128.524) (width 0.4) (layer F.Cu) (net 16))
 (segment (start 99.568 128.524) (end 99.568 131.42976) (width 0.4) (layer F.Cu) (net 16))
 (segment (start 99.568 131.42976) (end 96.4565 134.54126) (width 0.4) (layer F.Cu) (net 16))
 (segment (start 96.4565 148.1455) (end 93.726 150.876) (width 0.4) (layer F.Cu) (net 16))
 (segment (start 96.4565 134.54126) (end 96.4565 148.1455) (width 0.4) (layer F.Cu) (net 16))
 (segment (start 93.726 150.876) (end 93.345 150.876) (width 0.4) (layer F.Cu) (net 16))
 (segment (start 93.726 150.876) (end 93.6625 150.876) (width 0.25) (layer F.Cu) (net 16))
 (segment (start 96.012 81.788) (end 96.012 81.28) (width 0.4) (layer F.Cu) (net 17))
 (segment (start 95.504 80.772) (end 95.504 78.74) (width 0.4) (layer F.Cu) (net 17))
 (segment (start 96.012 81.28) (end 95.504 80.772) (width 0.4) (layer F.Cu) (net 17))
 (segment (start 94.488 77.724) (end 94.488 70.612) (width 0.4) (layer F.Cu) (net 17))
 (segment (start 95.504 78.74) (end 94.488 77.724) (width 0.4) (layer F.Cu) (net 17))
 (segment (start 92.231558 68.092659) (end 92.231558 68.355558) (width 0.4) (layer F.Cu) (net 17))
 (segment (start 92.231558 68.355558) (end 94.488 70.612) (width 0.4) (layer F.Cu) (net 17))
 (segment (start 96.012 81.788) (end 96.012 123.444) (width 0.4) (layer F.Cu) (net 17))
 (segment (start 96.012 123.444) (end 100.584 128.016) (width 0.4) (layer F.Cu) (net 17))
 (segment (start 100.584 128.016) (end 100.584 131.572) (width 0.4) (layer F.Cu) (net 17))
 (segment (start 100.584 131.572) (end 97.536 134.62) (width 0.4) (layer F.Cu) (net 17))
 (segment (start 97.536 134.62) (end 97.536 149.606) (width 0.4) (layer F.Cu) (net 17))
 (segment (start 97.536 149.606) (end 93.726 153.416) (width 0.4) (layer F.Cu) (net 17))
 (segment (start 93.726 153.416) (end 93.55836 153.416) (width 0.25) (layer F.Cu) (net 17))
 (segment (start 92.202 167.132) (end 93.726 168.656) (width 0.4) (layer F.Cu) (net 19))
 (segment (start 92.202 88.392) (end 92.202 167.132) (width 0.4) (layer F.Cu) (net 19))
 (segment (start 90.932 87.122) (end 92.202 88.392) (width 0.4) (layer F.Cu) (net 19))
 (segment (start 90.932 65.41008) (end 90.932 59.211897) (width 0.4) (layer F.Cu) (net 19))
 (segment (start 90.932 65.41008) (end 90.932 87.122) (width 0.4) (layer F.Cu) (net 19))
 (segment (start 90.932 59.211897) (end 92.221398 57.922499) (width 0.4) (layer F.Cu) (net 19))
 (segment (start 92.329 53.721) (end 92.2655 53.721) (width 0.4) (layer F.Cu) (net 20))
 (segment (start 90.297 60.96508) (end 90.297 54.929457) (width 0.4) (layer F.Cu) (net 20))
 (segment (start 90.297 54.929457) (end 92.297598 52.928859) (width 0.4) (layer F.Cu) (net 20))
 (segment (start 90.297 60.96508) (end 90.297 87.503) (width 0.4) (layer F.Cu) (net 20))
 (segment (start 90.297 87.503) (end 91.567 88.773) (width 0.4) (layer F.Cu) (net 20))
 (segment (start 91.567 88.773) (end 91.567 169.037) (width 0.4) (layer F.Cu) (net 20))
 (segment (start 91.567 169.037) (end 93.726 171.196) (width 0.4) (layer F.Cu) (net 20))
 (segment (start 92.180758 48.052059) (end 92.094981 48.052059) (width 0.4) (layer F.Cu) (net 21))
 (segment (start 92.094981 48.052059) (end 89.63152 50.51552) (width 0.4) (layer F.Cu) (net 21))
 (segment (start 89.63152 50.51552) (end 89.63152 87.706762) (width 0.4) (layer F.Cu) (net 21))
 (segment (start 89.63152 87.706762) (end 90.89136 88.966602) (width 0.4) (layer F.Cu) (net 21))
 (segment (start 90.89136 88.966602) (end 90.89136 170.90136) (width 0.4) (layer F.Cu) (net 21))
 (segment (start 90.89136 170.90136) (end 93.726 173.736) (width 0.4) (layer F.Cu) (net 21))
 (segment (start 97.028 77.724) (end 100.076 77.724) (width 0.4) (layer F.Cu) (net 6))
 (segment (start 100.076 77.724) (end 100.33 77.47) (width 0.4) (layer F.Cu) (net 6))
 (segment (start 100.076 77.724) (end 100.33 77.47) (width 0.4) (layer F.Cu) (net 6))
 (segment (start 97.028 72.644) (end 100.076 72.644) (width 0.4) (layer F.Cu) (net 7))
 (segment (start 100.076 72.644) (end 100.33 72.39) (width 0.4) (layer F.Cu) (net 7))
 (segment (start 97.028 67.564) (end 100.076 67.564) (width 0.4) (layer F.Cu) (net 8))
 (segment (start 100.076 67.564) (end 100.33 67.31) (width 0.4) (layer F.Cu) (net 8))
 (segment (start 97.1296 62.2554) (end 100.3046 62.2554) (width 0.4) (layer F.Cu) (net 9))
 (segment (start 100.3046 62.2554) (end 100.33 62.23) (width 0.4) (layer F.Cu) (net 9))
 (segment (start 97.19564 57.26684) (end 100.4824 57.26684) (width 0.4) (layer F.Cu) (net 10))
 (segment (start 98.4504 52.08016) (end 100.47732 52.08016) (width 0.4) (layer F.Cu) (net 11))
 (segment (start 98.44532 52.08524) (end 98.4504 52.08016) (width 0.4) (layer F.Cu) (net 11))
 (segment (start 97.11944 52.08524) (end 98.44532 52.08524) (width 0.4) (layer F.Cu) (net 11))
 (segment (start 100.41128 47.0916) (end 100.44684 47.05604) (width 0.6) (layer F.Cu) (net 12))
 (segment (start 97.19564 47.0916) (end 100.41128 47.0916) (width 0.4) (layer F.Cu) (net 12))
 (segment (start 97.0788 42.2148) (end 100.4062 42.2148) (width 0.4) (layer F.Cu) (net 13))
 (segment (start 100.4062 42.2148) (end 100.44684 42.25544) (width 0.6) (layer F.Cu) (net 13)))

